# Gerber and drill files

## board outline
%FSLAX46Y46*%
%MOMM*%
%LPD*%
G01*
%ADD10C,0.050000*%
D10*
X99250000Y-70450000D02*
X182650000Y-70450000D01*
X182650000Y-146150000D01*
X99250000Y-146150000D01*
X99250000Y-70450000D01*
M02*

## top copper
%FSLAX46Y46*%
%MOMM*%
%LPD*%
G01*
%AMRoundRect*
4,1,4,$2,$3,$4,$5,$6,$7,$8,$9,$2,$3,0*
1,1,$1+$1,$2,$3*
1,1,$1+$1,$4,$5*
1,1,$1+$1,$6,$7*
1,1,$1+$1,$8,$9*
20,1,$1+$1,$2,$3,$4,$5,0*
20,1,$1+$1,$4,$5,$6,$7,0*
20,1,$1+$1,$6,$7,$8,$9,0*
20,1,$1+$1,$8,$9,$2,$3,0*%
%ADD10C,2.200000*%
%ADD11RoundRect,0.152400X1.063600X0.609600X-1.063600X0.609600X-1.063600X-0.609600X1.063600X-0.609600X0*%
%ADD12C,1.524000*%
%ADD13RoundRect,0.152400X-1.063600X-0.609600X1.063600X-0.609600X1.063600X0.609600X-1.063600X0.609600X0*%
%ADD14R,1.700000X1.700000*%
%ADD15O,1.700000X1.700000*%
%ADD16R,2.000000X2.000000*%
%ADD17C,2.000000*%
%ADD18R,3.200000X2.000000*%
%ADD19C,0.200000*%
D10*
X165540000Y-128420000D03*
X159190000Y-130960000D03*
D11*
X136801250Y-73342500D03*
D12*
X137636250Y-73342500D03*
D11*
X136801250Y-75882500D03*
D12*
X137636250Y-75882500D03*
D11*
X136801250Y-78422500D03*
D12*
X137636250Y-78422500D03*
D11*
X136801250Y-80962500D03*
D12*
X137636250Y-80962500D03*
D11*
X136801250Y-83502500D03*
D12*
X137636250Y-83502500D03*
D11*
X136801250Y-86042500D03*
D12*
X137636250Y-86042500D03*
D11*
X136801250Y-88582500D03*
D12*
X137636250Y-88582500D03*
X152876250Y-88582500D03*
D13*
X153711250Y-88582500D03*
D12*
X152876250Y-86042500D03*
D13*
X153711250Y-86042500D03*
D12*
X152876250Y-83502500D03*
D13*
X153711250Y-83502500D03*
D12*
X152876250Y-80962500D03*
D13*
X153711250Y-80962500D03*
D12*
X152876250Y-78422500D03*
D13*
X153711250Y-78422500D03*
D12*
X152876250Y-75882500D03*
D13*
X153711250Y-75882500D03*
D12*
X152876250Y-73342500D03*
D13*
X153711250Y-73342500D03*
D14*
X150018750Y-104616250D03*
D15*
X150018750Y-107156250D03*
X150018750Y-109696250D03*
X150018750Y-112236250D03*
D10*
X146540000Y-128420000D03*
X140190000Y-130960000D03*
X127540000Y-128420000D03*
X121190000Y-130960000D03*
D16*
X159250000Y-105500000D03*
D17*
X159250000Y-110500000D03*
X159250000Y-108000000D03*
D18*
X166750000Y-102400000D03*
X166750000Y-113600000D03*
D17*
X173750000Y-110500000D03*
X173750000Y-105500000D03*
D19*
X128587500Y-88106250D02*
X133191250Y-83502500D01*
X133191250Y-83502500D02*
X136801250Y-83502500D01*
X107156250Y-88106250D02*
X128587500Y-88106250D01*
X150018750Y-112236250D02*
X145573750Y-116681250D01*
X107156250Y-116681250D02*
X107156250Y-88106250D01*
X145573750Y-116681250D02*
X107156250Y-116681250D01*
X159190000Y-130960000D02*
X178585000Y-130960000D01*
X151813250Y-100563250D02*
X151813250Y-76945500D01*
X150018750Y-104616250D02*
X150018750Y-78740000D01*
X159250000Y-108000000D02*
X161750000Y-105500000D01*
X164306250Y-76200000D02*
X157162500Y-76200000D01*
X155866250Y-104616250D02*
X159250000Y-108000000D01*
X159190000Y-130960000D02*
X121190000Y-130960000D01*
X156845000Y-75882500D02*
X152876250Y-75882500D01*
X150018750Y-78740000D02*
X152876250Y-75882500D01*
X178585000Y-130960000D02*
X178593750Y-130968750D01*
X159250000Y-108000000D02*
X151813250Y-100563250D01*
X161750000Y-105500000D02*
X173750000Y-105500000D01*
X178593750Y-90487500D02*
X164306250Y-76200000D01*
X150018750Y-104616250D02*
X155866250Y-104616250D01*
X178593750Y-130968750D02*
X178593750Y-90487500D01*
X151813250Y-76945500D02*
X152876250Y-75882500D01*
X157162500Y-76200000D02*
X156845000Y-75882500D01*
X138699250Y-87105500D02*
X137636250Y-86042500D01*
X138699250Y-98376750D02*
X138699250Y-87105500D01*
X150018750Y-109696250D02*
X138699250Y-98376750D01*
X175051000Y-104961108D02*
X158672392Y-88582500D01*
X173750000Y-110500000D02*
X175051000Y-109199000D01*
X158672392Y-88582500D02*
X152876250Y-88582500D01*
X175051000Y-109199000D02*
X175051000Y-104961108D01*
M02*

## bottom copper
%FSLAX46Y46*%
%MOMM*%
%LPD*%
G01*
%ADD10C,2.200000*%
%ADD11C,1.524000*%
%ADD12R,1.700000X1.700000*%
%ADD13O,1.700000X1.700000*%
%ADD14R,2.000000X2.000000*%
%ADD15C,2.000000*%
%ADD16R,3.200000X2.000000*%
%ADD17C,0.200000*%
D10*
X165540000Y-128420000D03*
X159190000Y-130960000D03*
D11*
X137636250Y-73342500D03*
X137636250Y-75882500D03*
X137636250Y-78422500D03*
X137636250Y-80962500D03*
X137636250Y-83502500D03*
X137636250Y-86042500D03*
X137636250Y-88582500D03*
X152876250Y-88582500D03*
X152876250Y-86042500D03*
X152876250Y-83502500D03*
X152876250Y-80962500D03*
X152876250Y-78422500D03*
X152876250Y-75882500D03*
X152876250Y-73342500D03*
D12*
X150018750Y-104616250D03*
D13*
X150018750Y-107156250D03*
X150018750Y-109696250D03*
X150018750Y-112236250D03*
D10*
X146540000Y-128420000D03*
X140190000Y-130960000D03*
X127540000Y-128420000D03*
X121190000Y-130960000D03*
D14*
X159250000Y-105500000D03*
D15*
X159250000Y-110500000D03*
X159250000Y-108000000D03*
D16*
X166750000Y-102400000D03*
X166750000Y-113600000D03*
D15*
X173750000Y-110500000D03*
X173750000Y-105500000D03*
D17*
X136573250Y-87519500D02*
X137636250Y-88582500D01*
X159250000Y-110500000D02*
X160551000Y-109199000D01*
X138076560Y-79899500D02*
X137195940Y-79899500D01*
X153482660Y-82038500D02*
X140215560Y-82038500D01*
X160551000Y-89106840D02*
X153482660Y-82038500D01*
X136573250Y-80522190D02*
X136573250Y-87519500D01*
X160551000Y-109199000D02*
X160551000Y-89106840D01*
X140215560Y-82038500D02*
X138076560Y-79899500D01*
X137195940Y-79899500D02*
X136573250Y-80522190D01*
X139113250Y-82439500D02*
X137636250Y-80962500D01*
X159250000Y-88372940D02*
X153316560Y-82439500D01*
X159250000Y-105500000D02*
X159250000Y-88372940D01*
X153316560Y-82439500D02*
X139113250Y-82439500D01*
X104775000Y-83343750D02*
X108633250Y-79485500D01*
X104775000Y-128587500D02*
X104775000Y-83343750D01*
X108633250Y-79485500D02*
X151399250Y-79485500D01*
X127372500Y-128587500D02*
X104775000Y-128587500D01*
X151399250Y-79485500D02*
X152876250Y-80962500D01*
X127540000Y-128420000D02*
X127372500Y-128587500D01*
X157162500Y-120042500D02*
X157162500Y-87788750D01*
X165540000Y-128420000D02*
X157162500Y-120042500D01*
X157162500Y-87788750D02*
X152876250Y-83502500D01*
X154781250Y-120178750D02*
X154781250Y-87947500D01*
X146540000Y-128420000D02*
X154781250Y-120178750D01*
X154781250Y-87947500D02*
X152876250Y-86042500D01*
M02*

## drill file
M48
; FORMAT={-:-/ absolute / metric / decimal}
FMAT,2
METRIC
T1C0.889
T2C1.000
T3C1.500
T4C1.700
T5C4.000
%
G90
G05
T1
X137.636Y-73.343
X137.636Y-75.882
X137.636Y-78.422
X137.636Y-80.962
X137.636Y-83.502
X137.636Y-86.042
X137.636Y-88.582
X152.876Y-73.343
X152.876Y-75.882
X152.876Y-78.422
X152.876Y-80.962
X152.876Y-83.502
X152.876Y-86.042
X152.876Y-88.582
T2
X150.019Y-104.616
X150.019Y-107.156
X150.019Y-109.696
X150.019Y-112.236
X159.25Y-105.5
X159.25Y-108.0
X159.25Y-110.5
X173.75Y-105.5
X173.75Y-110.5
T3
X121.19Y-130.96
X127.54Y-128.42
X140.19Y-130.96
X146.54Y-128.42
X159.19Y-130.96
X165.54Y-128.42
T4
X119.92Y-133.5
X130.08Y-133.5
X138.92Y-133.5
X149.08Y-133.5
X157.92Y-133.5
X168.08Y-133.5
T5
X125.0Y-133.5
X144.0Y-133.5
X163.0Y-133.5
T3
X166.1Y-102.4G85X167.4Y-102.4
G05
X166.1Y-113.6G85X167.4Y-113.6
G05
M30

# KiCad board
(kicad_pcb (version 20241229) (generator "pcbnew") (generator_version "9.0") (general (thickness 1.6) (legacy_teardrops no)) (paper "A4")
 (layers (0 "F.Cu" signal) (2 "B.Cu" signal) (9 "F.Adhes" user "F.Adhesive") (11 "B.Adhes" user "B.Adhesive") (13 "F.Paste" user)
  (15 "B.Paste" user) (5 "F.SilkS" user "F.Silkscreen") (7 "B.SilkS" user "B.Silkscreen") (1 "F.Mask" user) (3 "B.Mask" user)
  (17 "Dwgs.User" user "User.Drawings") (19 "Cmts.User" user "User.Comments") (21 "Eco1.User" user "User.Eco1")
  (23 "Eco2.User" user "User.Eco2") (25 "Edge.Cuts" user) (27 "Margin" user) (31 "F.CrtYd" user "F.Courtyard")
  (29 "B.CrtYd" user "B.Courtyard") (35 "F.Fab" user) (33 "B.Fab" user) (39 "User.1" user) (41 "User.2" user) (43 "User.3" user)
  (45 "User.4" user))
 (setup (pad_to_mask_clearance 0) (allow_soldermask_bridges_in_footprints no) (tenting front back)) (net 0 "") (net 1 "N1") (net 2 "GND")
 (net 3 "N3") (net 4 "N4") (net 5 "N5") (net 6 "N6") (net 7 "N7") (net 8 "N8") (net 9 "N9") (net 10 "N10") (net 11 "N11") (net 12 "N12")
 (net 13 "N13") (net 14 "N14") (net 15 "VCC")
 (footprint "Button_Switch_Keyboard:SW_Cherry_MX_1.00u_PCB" (layer "F.Cu") (at 165.54 128.42)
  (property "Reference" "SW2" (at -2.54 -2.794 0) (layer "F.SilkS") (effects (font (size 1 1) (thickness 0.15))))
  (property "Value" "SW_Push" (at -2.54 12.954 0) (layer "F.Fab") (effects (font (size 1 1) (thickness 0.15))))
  (pad "" np_thru_hole circle (at -7.62 5.08) (size 1.7 1.7) (drill 1.7) (layers "*.Cu" "*.Mask"))
  (pad "" np_thru_hole circle (at -2.54 5.08) (size 4 4) (drill 4) (layers "*.Cu" "*.Mask"))
  (pad "" np_thru_hole circle (at 2.54 5.08) (size 1.7 1.7) (drill 1.7) (layers "*.Cu" "*.Mask"))
  (pad "1" thru_hole circle (at 0 0) (size 2.2 2.2) (drill 1.5) (layers "*.Cu" "*.Mask") (remove_unused_layers no) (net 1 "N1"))
  (pad "2" thru_hole circle (at -6.35 2.54) (size 2.2 2.2) (drill 1.5) (layers "*.Cu" "*.Mask") (remove_unused_layers no) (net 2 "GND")))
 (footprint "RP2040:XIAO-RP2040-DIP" (layer "F.Cu") (at 145.25625 80.9625 90)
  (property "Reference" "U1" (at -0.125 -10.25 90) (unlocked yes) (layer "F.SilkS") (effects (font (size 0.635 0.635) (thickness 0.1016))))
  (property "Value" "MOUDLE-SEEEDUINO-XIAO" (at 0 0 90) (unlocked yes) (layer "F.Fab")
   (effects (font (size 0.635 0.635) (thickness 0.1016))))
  (pad "1" smd roundrect (at 7.62 -8.455 180) (size 2.432 1.524) (layers "F.Cu" "F.Mask") (roundrect_rratio 0.1) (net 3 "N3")
   (thermal_bridge_angle 45))
  (pad "1" thru_hole circle (at 7.62 -7.62 180) (size 1.524 1.524) (drill 0.889) (layers "*.Cu" "*.Mask") (remove_unused_layers no)
   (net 3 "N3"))
  (pad "2" smd roundrect (at 5.08 -8.455 180) (size 2.432 1.524) (layers "F.Cu" "F.Mask") (roundrect_rratio 0.1) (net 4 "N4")
   (thermal_bridge_angle 45))
  (pad "2" thru_hole circle (at 5.08 -7.62 180) (size 1.524 1.524) (drill 0.889) (layers "*.Cu" "*.Mask") (remove_unused_layers no)
   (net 4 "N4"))
  (pad "3" smd roundrect (at 2.54 -8.455 180) (size 2.432 1.524) (layers "F.Cu" "F.Mask") (roundrect_rratio 0.1) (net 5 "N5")
   (thermal_bridge_angle 45))
  (pad "3" thru_hole circle (at 2.54 -7.62 180) (size 1.524 1.524) (drill 0.889) (layers "*.Cu" "*.Mask") (remove_unused_layers no)
   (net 5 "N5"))
  (pad "4" smd roundrect (at 0 -8.455 180) (size 2.432 1.524) (layers "F.Cu" "F.Mask") (roundrect_rratio 0.1) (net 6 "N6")
   (thermal_bridge_angle 45))
  (pad "4" thru_hole circle (at 0 -7.62 180) (size 1.524 1.524) (drill 0.889) (layers "*.Cu" "*.Mask") (remove_unused_layers no)
   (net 6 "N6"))
  (pad "5" smd roundrect (at -2.54 -8.455 180) (size 2.432 1.524) (layers "F.Cu" "F.Mask") (roundrect_rratio 0.1) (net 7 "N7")
   (thermal_bridge_angle 45))
  (pad "5" thru_hole circle (at -2.54 -7.62 180) (size 1.524 1.524) (drill 0.889) (layers "*.Cu" "*.Mask") (remove_unused_layers no)
   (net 7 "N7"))
  (pad "6" smd roundrect (at -5.08 -8.455 180) (size 2.432 1.524) (layers "F.Cu" "F.Mask") (roundrect_rratio 0.1) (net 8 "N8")
   (thermal_bridge_angle 45))
  (pad "6" thru_hole circle (at -5.08 -7.62 180) (size 1.524 1.524) (drill 0.889) (layers "*.Cu" "*.Mask") (remove_unused_layers no)
   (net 8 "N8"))
  (pad "7" smd roundrect (at -7.62 -8.455 180) (size 2.432 1.524) (layers "F.Cu" "F.Mask") (roundrect_rratio 0.1) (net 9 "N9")
   (thermal_bridge_angle 45))
  (pad "7" thru_hole circle (at -7.62 -7.62 180) (size 1.524 1.524) (drill 0.889) (layers "*.Cu" "*.Mask") (remove_unused_layers no)
   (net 9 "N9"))
  (pad "8" thru_hole circle (at -7.62 7.62) (size 1.524 1.524) (drill 0.889) (layers "*.Cu" "*.Mask") (remove_unused_layers no)
   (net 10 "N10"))
  (pad "8" smd roundrect (at -7.62 8.455) (size 2.432 1.524) (layers "F.Cu" "F.Mask") (roundrect_rratio 0.1) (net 10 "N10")
   (thermal_bridge_angle 45))
  (pad "9" thru_hole circle (at -5.08 7.62) (size 1.524 1.524) (drill 0.889) (layers "*.Cu" "*.Mask") (remove_unused_layers no)
   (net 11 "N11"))
  (pad "9" smd roundrect (at -5.08 8.455) (size 2.432 1.524) (layers "F.Cu" "F.Mask") (roundrect_rratio 0.1) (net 11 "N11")
   (thermal_bridge_angle 45))
  (pad "10" thru_hole circle (at -2.54 7.62) (size 1.524 1.524) (drill 0.889) (layers "*.Cu" "*.Mask") (remove_unused_layers no)
   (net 1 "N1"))
  (pad "10" smd roundrect (at -2.54 8.455) (size 2.432 1.524) (layers "F.Cu" "F.Mask") (roundrect_rratio 0.1) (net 1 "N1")
   (thermal_bridge_angle 45))
  (pad "11" thru_hole circle (at 0 7.62) (size 1.524 1.524) (drill 0.889) (layers "*.Cu" "*.Mask") (remove_unused_layers no) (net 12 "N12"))
  (pad "11" smd roundrect (at 0 8.455) (size 2.432 1.524) (layers "F.Cu" "F.Mask") (roundrect_rratio 0.1) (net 12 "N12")
   (thermal_bridge_angle 45))
  (pad "12" thru_hole circle (at 2.54 7.62) (size 1.524 1.524) (drill 0.889) (layers "*.Cu" "*.Mask") (remove_unused_layers no)
   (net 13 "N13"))
  (pad "12" smd roundrect (at 2.54 8.455) (size 2.432 1.524) (layers "F.Cu" "F.Mask") (roundrect_rratio 0.1) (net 13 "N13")
   (thermal_bridge_angle 45))
  (pad "13" thru_hole circle (at 5.08 7.62) (size 1.524 1.524) (drill 0.889) (layers "*.Cu" "*.Mask") (remove_unused_layers no)
   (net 2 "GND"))
  (pad "13" smd roundrect (at 5.08 8.455) (size 2.432 1.524) (layers "F.Cu" "F.Mask") (roundrect_rratio 0.1) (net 2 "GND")
   (thermal_bridge_angle 45))
  (pad "14" thru_hole circle (at 7.62 7.62) (size 1.524 1.524) (drill 0.889) (layers "*.Cu" "*.Mask") (remove_unused_layers no)
   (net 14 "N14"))
  (pad "14" smd roundrect (at 7.62 8.455) (size 2.432 1.524) (layers "F.Cu" "F.Mask") (roundrect_rratio 0.1) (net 14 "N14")
   (thermal_bridge_angle 45)))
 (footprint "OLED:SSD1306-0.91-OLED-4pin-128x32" (layer "F.Cu") (at 113.51875 102.42625)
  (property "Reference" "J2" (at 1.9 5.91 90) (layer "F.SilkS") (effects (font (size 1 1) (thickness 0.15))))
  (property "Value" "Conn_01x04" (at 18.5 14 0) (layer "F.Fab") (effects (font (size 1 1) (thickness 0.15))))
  (pad "1" thru_hole rect (at 36.5 2.19) (size 1.7 1.7) (drill 1) (layers "*.Cu" "*.Mask") (remove_unused_layers no) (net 2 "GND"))
  (pad "2" thru_hole oval (at 36.5 4.73) (size 1.7 1.7) (drill 1) (layers "*.Cu" "*.Mask") (remove_unused_layers no) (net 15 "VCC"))
  (pad "3" thru_hole oval (at 36.5 7.27) (size 1.7 1.7) (drill 1) (layers "*.Cu" "*.Mask") (remove_unused_layers no) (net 8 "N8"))
  (pad "4" thru_hole oval (at 36.5 9.81) (size 1.7 1.7) (drill 1) (layers "*.Cu" "*.Mask") (remove_unused_layers no) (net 7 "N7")))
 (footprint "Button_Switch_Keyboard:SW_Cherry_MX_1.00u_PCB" (layer "F.Cu") (at 146.54 128.42)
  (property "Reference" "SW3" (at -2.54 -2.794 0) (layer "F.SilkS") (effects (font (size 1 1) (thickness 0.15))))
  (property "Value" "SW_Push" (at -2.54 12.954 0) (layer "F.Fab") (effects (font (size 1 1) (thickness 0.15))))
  (pad "" np_thru_hole circle (at -7.62 5.08) (size 1.7 1.7) (drill 1.7) (layers "*.Cu" "*.Mask"))
  (pad "" np_thru_hole circle (at -2.54 5.08) (size 4 4) (drill 4) (layers "*.Cu" "*.Mask"))
  (pad "" np_thru_hole circle (at 2.54 5.08) (size 1.7 1.7) (drill 1.7) (layers "*.Cu" "*.Mask"))
  (pad "1" thru_hole circle (at 0 0) (size 2.2 2.2) (drill 1.5) (layers "*.Cu" "*.Mask") (remove_unused_layers no) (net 11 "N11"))
  (pad "2" thru_hole circle (at -6.35 2.54) (size 2.2 2.2) (drill 1.5) (layers "*.Cu" "*.Mask") (remove_unused_layers no) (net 2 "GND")))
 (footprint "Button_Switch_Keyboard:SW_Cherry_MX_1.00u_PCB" (layer "F.Cu") (at 127.54 128.42)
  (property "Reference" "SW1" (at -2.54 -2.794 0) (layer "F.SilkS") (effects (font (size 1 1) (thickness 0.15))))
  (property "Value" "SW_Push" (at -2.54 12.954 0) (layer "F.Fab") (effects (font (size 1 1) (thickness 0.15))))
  (pad "" np_thru_hole circle (at -7.62 5.08) (size 1.7 1.7) (drill 1.7) (layers "*.Cu" "*.Mask"))
  (pad "" np_thru_hole circle (at -2.54 5.08) (size 4 4) (drill 4) (layers "*.Cu" "*.Mask"))
  (pad "" np_thru_hole circle (at 2.54 5.08) (size 1.7 1.7) (drill 1.7) (layers "*.Cu" "*.Mask"))
  (pad "1" thru_hole circle (at 0 0) (size 2.2 2.2) (drill 1.5) (layers "*.Cu" "*.Mask") (remove_unused_layers no) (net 12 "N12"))
  (pad "2" thru_hole circle (at -6.35 2.54) (size 2.2 2.2) (drill 1.5) (layers "*.Cu" "*.Mask") (remove_unused_layers no) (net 2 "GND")))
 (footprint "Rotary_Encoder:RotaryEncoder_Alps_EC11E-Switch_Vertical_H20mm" (layer "F.Cu") (at 159.25 105.5)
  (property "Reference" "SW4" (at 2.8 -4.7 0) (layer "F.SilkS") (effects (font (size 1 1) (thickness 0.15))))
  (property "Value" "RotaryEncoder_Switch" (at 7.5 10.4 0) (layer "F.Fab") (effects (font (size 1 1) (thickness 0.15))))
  (pad "A" thru_hole rect (at 0 0) (size 2 2) (drill 1) (layers "*.Cu" "*.Mask") (remove_unused_layers no) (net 6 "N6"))
  (pad "B" thru_hole circle (at 0 5) (size 2 2) (drill 1) (layers "*.Cu" "*.Mask") (remove_unused_layers no) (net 9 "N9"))
  (pad "C" thru_hole circle (at 0 2.5) (size 2 2) (drill 1) (layers "*.Cu" "*.Mask") (remove_unused_layers no) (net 2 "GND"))
  (pad "MP" thru_hole rect (at 7.5 -3.1) (size 3.2 2) (drill oval 2.8 1.5) (layers "*.Cu" "*.Mask") (remove_unused_layers no))
  (pad "MP" thru_hole rect (at 7.5 8.1) (size 3.2 2) (drill oval 2.8 1.5) (layers "*.Cu" "*.Mask") (remove_unused_layers no))
  (pad "S1" thru_hole circle (at 14.5 5) (size 2 2) (drill 1) (layers "*.Cu" "*.Mask") (remove_unused_layers no) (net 10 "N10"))
  (pad "S2" thru_hole circle (at 14.5 0) (size 2 2) (drill 1) (layers "*.Cu" "*.Mask") (remove_unused_layers no) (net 2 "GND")))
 (gr_rect (start 99.25 70.45) (end 182.65 146.15) (stroke (width 0.05) (type default)) (fill no) (layer "Edge.Cuts"))
 (segment (start 128.5875 88.10625) (end 133.19125 83.5025) (width 0.2) (layer "F.Cu") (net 7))
 (segment (start 133.19125 83.5025) (end 136.80125 83.5025) (width 0.2) (layer "F.Cu") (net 7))
 (segment (start 107.15625 88.10625) (end 128.5875 88.10625) (width 0.2) (layer "F.Cu") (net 7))
 (segment (start 150.01875 112.23625) (end 145.57375 116.68125) (width 0.2) (layer "F.Cu") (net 7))
 (segment (start 107.15625 116.68125) (end 107.15625 88.10625) (width 0.2) (layer "F.Cu") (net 7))
 (segment (start 145.57375 116.68125) (end 107.15625 116.68125) (width 0.2) (layer "F.Cu") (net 7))
 (segment (start 159.19 130.96) (end 178.585 130.96) (width 0.2) (layer "F.Cu") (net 2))
 (segment (start 151.81325 100.56325) (end 151.81325 76.9455) (width 0.2) (layer "F.Cu") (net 2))
 (segment (start 150.01875 104.61625) (end 150.01875 78.74) (width 0.2) (layer "F.Cu") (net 2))
 (segment (start 159.25 108) (end 161.75 105.5) (width 0.2) (layer "F.Cu") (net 2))
 (segment (start 164.30625 76.2) (end 157.1625 76.2) (width 0.2) (layer "F.Cu") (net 2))
 (segment (start 155.86625 104.61625) (end 159.25 108) (width 0.2) (layer "F.Cu") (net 2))
 (segment (start 159.19 130.96) (end 121.19 130.96) (width 0.2) (layer "F.Cu") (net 2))
 (segment (start 156.845 75.8825) (end 152.87625 75.8825) (width 0.2) (layer "F.Cu") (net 2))
 (segment (start 150.01875 78.74) (end 152.87625 75.8825) (width 0.2) (layer "F.Cu") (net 2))
 (segment (start 178.585 130.96) (end 178.59375 130.96875) (width 0.2) (layer "F.Cu") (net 2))
 (segment (start 159.25 108) (end 151.81325 100.56325) (width 0.2) (layer "F.Cu") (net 2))
 (segment (start 161.75 105.5) (end 173.75 105.5) (width 0.2) (layer "F.Cu") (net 2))
 (segment (start 178.59375 90.4875) (end 164.30625 76.2) (width 0.2) (layer "F.Cu") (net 2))
 (segment (start 150.01875 104.61625) (end 155.86625 104.61625) (width 0.2) (layer "F.Cu") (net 2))
 (segment (start 178.59375 130.96875) (end 178.59375 90.4875) (width 0.2) (layer "F.Cu") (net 2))
 (segment (start 151.81325 76.9455) (end 152.87625 75.8825) (width 0.2) (layer "F.Cu") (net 2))
 (segment (start 157.1625 76.2) (end 156.845 75.8825) (width 0.2) (layer "F.Cu") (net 2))
 (segment (start 138.69925 87.1055) (end 137.63625 86.0425) (width 0.2) (layer "F.Cu") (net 8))
 (segment (start 138.69925 98.37675) (end 138.69925 87.1055) (width 0.2) (layer "F.Cu") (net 8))
 (segment (start 150.01875 109.69625) (end 138.69925 98.37675) (width 0.2) (layer "F.Cu") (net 8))
 (segment (start 136.57325 87.5195) (end 137.63625 88.5825) (width 0.2) (layer "B.Cu") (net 9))
 (segment (start 159.25 110.5) (end 160.551 109.199) (width 0.2) (layer "B.Cu") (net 9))
 (segment (start 138.07656 79.8995) (end 137.19594 79.8995) (width 0.2) (layer "B.Cu") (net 9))
 (segment (start 153.48266 82.0385) (end 140.21556 82.0385) (width 0.2) (layer "B.Cu") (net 9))
 (segment (start 160.551 89.10684) (end 153.48266 82.0385) (width 0.2) (layer "B.Cu") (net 9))
 (segment (start 136.57325 80.52219) (end 136.57325 87.5195) (width 0.2) (layer "B.Cu") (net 9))
 (segment (start 160.551 109.199) (end 160.551 89.10684) (width 0.2) (layer "B.Cu") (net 9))
 (segment (start 140.21556 82.0385) (end 138.07656 79.8995) (width 0.2) (layer "B.Cu") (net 9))
 (segment (start 137.19594 79.8995) (end 136.57325 80.52219) (width 0.2) (layer "B.Cu") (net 9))
 (segment (start 139.11325 82.4395) (end 137.63625 80.9625) (width 0.2) (layer "B.Cu") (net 6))
 (segment (start 159.25 88.37294) (end 153.31656 82.4395) (width 0.2) (layer "B.Cu") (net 6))
 (segment (start 159.25 105.5) (end 159.25 88.37294) (width 0.2) (layer "B.Cu") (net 6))
 (segment (start 153.31656 82.4395) (end 139.11325 82.4395) (width 0.2) (layer "B.Cu") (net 6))
 (segment (start 175.051 104.961108) (end 158.672392 88.5825) (width 0.2) (layer "F.Cu") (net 10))
 (segment (start 173.75 110.5) (end 175.051 109.199) (width 0.2) (layer "F.Cu") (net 10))
 (segment (start 158.672392 88.5825) (end 152.87625 88.5825) (width 0.2) (layer "F.Cu") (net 10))
 (segment (start 175.051 109.199) (end 175.051 104.961108) (width 0.2) (layer "F.Cu") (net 10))
 (segment (start 104.775 83.34375) (end 108.63325 79.4855) (width 0.2) (layer "B.Cu") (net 12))
 (segment (start 104.775 128.5875) (end 104.775 83.34375) (width 0.2) (layer "B.Cu") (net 12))
 (segment (start 108.63325 79.4855) (end 151.39925 79.4855) (width 0.2) (layer "B.Cu") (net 12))
 (segment (start 127.3725 128.5875) (end 104.775 128.5875) (width 0.2) (layer "B.Cu") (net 12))
 (segment (start 151.39925 79.4855) (end 152.87625 80.9625) (width 0.2) (layer "B.Cu") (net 12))
 (segment (start 127.54 128.42) (end 127.3725 128.5875) (width 0.2) (layer "B.Cu") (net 12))
 (segment (start 157.1625 120.0425) (end 157.1625 87.78875) (width 0.2) (layer "B.Cu") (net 1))
 (segment (start 165.54 128.42) (end 157.1625 120.0425) (width 0.2) (layer "B.Cu") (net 1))
 (segment (start 157.1625 87.78875) (end 152.87625 83.5025) (width 0.2) (layer "B.Cu") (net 1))
 (segment (start 154.78125 120.17875) (end 154.78125 87.9475) (width 0.2) (layer "B.Cu") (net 11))
 (segment (start 146.54 128.42) (end 154.78125 120.17875) (width 0.2) (layer "B.Cu") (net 11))
 (segment (start 154.78125 87.9475) (end 152.87625 86.0425) (width 0.2) (layer "B.Cu") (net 11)))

